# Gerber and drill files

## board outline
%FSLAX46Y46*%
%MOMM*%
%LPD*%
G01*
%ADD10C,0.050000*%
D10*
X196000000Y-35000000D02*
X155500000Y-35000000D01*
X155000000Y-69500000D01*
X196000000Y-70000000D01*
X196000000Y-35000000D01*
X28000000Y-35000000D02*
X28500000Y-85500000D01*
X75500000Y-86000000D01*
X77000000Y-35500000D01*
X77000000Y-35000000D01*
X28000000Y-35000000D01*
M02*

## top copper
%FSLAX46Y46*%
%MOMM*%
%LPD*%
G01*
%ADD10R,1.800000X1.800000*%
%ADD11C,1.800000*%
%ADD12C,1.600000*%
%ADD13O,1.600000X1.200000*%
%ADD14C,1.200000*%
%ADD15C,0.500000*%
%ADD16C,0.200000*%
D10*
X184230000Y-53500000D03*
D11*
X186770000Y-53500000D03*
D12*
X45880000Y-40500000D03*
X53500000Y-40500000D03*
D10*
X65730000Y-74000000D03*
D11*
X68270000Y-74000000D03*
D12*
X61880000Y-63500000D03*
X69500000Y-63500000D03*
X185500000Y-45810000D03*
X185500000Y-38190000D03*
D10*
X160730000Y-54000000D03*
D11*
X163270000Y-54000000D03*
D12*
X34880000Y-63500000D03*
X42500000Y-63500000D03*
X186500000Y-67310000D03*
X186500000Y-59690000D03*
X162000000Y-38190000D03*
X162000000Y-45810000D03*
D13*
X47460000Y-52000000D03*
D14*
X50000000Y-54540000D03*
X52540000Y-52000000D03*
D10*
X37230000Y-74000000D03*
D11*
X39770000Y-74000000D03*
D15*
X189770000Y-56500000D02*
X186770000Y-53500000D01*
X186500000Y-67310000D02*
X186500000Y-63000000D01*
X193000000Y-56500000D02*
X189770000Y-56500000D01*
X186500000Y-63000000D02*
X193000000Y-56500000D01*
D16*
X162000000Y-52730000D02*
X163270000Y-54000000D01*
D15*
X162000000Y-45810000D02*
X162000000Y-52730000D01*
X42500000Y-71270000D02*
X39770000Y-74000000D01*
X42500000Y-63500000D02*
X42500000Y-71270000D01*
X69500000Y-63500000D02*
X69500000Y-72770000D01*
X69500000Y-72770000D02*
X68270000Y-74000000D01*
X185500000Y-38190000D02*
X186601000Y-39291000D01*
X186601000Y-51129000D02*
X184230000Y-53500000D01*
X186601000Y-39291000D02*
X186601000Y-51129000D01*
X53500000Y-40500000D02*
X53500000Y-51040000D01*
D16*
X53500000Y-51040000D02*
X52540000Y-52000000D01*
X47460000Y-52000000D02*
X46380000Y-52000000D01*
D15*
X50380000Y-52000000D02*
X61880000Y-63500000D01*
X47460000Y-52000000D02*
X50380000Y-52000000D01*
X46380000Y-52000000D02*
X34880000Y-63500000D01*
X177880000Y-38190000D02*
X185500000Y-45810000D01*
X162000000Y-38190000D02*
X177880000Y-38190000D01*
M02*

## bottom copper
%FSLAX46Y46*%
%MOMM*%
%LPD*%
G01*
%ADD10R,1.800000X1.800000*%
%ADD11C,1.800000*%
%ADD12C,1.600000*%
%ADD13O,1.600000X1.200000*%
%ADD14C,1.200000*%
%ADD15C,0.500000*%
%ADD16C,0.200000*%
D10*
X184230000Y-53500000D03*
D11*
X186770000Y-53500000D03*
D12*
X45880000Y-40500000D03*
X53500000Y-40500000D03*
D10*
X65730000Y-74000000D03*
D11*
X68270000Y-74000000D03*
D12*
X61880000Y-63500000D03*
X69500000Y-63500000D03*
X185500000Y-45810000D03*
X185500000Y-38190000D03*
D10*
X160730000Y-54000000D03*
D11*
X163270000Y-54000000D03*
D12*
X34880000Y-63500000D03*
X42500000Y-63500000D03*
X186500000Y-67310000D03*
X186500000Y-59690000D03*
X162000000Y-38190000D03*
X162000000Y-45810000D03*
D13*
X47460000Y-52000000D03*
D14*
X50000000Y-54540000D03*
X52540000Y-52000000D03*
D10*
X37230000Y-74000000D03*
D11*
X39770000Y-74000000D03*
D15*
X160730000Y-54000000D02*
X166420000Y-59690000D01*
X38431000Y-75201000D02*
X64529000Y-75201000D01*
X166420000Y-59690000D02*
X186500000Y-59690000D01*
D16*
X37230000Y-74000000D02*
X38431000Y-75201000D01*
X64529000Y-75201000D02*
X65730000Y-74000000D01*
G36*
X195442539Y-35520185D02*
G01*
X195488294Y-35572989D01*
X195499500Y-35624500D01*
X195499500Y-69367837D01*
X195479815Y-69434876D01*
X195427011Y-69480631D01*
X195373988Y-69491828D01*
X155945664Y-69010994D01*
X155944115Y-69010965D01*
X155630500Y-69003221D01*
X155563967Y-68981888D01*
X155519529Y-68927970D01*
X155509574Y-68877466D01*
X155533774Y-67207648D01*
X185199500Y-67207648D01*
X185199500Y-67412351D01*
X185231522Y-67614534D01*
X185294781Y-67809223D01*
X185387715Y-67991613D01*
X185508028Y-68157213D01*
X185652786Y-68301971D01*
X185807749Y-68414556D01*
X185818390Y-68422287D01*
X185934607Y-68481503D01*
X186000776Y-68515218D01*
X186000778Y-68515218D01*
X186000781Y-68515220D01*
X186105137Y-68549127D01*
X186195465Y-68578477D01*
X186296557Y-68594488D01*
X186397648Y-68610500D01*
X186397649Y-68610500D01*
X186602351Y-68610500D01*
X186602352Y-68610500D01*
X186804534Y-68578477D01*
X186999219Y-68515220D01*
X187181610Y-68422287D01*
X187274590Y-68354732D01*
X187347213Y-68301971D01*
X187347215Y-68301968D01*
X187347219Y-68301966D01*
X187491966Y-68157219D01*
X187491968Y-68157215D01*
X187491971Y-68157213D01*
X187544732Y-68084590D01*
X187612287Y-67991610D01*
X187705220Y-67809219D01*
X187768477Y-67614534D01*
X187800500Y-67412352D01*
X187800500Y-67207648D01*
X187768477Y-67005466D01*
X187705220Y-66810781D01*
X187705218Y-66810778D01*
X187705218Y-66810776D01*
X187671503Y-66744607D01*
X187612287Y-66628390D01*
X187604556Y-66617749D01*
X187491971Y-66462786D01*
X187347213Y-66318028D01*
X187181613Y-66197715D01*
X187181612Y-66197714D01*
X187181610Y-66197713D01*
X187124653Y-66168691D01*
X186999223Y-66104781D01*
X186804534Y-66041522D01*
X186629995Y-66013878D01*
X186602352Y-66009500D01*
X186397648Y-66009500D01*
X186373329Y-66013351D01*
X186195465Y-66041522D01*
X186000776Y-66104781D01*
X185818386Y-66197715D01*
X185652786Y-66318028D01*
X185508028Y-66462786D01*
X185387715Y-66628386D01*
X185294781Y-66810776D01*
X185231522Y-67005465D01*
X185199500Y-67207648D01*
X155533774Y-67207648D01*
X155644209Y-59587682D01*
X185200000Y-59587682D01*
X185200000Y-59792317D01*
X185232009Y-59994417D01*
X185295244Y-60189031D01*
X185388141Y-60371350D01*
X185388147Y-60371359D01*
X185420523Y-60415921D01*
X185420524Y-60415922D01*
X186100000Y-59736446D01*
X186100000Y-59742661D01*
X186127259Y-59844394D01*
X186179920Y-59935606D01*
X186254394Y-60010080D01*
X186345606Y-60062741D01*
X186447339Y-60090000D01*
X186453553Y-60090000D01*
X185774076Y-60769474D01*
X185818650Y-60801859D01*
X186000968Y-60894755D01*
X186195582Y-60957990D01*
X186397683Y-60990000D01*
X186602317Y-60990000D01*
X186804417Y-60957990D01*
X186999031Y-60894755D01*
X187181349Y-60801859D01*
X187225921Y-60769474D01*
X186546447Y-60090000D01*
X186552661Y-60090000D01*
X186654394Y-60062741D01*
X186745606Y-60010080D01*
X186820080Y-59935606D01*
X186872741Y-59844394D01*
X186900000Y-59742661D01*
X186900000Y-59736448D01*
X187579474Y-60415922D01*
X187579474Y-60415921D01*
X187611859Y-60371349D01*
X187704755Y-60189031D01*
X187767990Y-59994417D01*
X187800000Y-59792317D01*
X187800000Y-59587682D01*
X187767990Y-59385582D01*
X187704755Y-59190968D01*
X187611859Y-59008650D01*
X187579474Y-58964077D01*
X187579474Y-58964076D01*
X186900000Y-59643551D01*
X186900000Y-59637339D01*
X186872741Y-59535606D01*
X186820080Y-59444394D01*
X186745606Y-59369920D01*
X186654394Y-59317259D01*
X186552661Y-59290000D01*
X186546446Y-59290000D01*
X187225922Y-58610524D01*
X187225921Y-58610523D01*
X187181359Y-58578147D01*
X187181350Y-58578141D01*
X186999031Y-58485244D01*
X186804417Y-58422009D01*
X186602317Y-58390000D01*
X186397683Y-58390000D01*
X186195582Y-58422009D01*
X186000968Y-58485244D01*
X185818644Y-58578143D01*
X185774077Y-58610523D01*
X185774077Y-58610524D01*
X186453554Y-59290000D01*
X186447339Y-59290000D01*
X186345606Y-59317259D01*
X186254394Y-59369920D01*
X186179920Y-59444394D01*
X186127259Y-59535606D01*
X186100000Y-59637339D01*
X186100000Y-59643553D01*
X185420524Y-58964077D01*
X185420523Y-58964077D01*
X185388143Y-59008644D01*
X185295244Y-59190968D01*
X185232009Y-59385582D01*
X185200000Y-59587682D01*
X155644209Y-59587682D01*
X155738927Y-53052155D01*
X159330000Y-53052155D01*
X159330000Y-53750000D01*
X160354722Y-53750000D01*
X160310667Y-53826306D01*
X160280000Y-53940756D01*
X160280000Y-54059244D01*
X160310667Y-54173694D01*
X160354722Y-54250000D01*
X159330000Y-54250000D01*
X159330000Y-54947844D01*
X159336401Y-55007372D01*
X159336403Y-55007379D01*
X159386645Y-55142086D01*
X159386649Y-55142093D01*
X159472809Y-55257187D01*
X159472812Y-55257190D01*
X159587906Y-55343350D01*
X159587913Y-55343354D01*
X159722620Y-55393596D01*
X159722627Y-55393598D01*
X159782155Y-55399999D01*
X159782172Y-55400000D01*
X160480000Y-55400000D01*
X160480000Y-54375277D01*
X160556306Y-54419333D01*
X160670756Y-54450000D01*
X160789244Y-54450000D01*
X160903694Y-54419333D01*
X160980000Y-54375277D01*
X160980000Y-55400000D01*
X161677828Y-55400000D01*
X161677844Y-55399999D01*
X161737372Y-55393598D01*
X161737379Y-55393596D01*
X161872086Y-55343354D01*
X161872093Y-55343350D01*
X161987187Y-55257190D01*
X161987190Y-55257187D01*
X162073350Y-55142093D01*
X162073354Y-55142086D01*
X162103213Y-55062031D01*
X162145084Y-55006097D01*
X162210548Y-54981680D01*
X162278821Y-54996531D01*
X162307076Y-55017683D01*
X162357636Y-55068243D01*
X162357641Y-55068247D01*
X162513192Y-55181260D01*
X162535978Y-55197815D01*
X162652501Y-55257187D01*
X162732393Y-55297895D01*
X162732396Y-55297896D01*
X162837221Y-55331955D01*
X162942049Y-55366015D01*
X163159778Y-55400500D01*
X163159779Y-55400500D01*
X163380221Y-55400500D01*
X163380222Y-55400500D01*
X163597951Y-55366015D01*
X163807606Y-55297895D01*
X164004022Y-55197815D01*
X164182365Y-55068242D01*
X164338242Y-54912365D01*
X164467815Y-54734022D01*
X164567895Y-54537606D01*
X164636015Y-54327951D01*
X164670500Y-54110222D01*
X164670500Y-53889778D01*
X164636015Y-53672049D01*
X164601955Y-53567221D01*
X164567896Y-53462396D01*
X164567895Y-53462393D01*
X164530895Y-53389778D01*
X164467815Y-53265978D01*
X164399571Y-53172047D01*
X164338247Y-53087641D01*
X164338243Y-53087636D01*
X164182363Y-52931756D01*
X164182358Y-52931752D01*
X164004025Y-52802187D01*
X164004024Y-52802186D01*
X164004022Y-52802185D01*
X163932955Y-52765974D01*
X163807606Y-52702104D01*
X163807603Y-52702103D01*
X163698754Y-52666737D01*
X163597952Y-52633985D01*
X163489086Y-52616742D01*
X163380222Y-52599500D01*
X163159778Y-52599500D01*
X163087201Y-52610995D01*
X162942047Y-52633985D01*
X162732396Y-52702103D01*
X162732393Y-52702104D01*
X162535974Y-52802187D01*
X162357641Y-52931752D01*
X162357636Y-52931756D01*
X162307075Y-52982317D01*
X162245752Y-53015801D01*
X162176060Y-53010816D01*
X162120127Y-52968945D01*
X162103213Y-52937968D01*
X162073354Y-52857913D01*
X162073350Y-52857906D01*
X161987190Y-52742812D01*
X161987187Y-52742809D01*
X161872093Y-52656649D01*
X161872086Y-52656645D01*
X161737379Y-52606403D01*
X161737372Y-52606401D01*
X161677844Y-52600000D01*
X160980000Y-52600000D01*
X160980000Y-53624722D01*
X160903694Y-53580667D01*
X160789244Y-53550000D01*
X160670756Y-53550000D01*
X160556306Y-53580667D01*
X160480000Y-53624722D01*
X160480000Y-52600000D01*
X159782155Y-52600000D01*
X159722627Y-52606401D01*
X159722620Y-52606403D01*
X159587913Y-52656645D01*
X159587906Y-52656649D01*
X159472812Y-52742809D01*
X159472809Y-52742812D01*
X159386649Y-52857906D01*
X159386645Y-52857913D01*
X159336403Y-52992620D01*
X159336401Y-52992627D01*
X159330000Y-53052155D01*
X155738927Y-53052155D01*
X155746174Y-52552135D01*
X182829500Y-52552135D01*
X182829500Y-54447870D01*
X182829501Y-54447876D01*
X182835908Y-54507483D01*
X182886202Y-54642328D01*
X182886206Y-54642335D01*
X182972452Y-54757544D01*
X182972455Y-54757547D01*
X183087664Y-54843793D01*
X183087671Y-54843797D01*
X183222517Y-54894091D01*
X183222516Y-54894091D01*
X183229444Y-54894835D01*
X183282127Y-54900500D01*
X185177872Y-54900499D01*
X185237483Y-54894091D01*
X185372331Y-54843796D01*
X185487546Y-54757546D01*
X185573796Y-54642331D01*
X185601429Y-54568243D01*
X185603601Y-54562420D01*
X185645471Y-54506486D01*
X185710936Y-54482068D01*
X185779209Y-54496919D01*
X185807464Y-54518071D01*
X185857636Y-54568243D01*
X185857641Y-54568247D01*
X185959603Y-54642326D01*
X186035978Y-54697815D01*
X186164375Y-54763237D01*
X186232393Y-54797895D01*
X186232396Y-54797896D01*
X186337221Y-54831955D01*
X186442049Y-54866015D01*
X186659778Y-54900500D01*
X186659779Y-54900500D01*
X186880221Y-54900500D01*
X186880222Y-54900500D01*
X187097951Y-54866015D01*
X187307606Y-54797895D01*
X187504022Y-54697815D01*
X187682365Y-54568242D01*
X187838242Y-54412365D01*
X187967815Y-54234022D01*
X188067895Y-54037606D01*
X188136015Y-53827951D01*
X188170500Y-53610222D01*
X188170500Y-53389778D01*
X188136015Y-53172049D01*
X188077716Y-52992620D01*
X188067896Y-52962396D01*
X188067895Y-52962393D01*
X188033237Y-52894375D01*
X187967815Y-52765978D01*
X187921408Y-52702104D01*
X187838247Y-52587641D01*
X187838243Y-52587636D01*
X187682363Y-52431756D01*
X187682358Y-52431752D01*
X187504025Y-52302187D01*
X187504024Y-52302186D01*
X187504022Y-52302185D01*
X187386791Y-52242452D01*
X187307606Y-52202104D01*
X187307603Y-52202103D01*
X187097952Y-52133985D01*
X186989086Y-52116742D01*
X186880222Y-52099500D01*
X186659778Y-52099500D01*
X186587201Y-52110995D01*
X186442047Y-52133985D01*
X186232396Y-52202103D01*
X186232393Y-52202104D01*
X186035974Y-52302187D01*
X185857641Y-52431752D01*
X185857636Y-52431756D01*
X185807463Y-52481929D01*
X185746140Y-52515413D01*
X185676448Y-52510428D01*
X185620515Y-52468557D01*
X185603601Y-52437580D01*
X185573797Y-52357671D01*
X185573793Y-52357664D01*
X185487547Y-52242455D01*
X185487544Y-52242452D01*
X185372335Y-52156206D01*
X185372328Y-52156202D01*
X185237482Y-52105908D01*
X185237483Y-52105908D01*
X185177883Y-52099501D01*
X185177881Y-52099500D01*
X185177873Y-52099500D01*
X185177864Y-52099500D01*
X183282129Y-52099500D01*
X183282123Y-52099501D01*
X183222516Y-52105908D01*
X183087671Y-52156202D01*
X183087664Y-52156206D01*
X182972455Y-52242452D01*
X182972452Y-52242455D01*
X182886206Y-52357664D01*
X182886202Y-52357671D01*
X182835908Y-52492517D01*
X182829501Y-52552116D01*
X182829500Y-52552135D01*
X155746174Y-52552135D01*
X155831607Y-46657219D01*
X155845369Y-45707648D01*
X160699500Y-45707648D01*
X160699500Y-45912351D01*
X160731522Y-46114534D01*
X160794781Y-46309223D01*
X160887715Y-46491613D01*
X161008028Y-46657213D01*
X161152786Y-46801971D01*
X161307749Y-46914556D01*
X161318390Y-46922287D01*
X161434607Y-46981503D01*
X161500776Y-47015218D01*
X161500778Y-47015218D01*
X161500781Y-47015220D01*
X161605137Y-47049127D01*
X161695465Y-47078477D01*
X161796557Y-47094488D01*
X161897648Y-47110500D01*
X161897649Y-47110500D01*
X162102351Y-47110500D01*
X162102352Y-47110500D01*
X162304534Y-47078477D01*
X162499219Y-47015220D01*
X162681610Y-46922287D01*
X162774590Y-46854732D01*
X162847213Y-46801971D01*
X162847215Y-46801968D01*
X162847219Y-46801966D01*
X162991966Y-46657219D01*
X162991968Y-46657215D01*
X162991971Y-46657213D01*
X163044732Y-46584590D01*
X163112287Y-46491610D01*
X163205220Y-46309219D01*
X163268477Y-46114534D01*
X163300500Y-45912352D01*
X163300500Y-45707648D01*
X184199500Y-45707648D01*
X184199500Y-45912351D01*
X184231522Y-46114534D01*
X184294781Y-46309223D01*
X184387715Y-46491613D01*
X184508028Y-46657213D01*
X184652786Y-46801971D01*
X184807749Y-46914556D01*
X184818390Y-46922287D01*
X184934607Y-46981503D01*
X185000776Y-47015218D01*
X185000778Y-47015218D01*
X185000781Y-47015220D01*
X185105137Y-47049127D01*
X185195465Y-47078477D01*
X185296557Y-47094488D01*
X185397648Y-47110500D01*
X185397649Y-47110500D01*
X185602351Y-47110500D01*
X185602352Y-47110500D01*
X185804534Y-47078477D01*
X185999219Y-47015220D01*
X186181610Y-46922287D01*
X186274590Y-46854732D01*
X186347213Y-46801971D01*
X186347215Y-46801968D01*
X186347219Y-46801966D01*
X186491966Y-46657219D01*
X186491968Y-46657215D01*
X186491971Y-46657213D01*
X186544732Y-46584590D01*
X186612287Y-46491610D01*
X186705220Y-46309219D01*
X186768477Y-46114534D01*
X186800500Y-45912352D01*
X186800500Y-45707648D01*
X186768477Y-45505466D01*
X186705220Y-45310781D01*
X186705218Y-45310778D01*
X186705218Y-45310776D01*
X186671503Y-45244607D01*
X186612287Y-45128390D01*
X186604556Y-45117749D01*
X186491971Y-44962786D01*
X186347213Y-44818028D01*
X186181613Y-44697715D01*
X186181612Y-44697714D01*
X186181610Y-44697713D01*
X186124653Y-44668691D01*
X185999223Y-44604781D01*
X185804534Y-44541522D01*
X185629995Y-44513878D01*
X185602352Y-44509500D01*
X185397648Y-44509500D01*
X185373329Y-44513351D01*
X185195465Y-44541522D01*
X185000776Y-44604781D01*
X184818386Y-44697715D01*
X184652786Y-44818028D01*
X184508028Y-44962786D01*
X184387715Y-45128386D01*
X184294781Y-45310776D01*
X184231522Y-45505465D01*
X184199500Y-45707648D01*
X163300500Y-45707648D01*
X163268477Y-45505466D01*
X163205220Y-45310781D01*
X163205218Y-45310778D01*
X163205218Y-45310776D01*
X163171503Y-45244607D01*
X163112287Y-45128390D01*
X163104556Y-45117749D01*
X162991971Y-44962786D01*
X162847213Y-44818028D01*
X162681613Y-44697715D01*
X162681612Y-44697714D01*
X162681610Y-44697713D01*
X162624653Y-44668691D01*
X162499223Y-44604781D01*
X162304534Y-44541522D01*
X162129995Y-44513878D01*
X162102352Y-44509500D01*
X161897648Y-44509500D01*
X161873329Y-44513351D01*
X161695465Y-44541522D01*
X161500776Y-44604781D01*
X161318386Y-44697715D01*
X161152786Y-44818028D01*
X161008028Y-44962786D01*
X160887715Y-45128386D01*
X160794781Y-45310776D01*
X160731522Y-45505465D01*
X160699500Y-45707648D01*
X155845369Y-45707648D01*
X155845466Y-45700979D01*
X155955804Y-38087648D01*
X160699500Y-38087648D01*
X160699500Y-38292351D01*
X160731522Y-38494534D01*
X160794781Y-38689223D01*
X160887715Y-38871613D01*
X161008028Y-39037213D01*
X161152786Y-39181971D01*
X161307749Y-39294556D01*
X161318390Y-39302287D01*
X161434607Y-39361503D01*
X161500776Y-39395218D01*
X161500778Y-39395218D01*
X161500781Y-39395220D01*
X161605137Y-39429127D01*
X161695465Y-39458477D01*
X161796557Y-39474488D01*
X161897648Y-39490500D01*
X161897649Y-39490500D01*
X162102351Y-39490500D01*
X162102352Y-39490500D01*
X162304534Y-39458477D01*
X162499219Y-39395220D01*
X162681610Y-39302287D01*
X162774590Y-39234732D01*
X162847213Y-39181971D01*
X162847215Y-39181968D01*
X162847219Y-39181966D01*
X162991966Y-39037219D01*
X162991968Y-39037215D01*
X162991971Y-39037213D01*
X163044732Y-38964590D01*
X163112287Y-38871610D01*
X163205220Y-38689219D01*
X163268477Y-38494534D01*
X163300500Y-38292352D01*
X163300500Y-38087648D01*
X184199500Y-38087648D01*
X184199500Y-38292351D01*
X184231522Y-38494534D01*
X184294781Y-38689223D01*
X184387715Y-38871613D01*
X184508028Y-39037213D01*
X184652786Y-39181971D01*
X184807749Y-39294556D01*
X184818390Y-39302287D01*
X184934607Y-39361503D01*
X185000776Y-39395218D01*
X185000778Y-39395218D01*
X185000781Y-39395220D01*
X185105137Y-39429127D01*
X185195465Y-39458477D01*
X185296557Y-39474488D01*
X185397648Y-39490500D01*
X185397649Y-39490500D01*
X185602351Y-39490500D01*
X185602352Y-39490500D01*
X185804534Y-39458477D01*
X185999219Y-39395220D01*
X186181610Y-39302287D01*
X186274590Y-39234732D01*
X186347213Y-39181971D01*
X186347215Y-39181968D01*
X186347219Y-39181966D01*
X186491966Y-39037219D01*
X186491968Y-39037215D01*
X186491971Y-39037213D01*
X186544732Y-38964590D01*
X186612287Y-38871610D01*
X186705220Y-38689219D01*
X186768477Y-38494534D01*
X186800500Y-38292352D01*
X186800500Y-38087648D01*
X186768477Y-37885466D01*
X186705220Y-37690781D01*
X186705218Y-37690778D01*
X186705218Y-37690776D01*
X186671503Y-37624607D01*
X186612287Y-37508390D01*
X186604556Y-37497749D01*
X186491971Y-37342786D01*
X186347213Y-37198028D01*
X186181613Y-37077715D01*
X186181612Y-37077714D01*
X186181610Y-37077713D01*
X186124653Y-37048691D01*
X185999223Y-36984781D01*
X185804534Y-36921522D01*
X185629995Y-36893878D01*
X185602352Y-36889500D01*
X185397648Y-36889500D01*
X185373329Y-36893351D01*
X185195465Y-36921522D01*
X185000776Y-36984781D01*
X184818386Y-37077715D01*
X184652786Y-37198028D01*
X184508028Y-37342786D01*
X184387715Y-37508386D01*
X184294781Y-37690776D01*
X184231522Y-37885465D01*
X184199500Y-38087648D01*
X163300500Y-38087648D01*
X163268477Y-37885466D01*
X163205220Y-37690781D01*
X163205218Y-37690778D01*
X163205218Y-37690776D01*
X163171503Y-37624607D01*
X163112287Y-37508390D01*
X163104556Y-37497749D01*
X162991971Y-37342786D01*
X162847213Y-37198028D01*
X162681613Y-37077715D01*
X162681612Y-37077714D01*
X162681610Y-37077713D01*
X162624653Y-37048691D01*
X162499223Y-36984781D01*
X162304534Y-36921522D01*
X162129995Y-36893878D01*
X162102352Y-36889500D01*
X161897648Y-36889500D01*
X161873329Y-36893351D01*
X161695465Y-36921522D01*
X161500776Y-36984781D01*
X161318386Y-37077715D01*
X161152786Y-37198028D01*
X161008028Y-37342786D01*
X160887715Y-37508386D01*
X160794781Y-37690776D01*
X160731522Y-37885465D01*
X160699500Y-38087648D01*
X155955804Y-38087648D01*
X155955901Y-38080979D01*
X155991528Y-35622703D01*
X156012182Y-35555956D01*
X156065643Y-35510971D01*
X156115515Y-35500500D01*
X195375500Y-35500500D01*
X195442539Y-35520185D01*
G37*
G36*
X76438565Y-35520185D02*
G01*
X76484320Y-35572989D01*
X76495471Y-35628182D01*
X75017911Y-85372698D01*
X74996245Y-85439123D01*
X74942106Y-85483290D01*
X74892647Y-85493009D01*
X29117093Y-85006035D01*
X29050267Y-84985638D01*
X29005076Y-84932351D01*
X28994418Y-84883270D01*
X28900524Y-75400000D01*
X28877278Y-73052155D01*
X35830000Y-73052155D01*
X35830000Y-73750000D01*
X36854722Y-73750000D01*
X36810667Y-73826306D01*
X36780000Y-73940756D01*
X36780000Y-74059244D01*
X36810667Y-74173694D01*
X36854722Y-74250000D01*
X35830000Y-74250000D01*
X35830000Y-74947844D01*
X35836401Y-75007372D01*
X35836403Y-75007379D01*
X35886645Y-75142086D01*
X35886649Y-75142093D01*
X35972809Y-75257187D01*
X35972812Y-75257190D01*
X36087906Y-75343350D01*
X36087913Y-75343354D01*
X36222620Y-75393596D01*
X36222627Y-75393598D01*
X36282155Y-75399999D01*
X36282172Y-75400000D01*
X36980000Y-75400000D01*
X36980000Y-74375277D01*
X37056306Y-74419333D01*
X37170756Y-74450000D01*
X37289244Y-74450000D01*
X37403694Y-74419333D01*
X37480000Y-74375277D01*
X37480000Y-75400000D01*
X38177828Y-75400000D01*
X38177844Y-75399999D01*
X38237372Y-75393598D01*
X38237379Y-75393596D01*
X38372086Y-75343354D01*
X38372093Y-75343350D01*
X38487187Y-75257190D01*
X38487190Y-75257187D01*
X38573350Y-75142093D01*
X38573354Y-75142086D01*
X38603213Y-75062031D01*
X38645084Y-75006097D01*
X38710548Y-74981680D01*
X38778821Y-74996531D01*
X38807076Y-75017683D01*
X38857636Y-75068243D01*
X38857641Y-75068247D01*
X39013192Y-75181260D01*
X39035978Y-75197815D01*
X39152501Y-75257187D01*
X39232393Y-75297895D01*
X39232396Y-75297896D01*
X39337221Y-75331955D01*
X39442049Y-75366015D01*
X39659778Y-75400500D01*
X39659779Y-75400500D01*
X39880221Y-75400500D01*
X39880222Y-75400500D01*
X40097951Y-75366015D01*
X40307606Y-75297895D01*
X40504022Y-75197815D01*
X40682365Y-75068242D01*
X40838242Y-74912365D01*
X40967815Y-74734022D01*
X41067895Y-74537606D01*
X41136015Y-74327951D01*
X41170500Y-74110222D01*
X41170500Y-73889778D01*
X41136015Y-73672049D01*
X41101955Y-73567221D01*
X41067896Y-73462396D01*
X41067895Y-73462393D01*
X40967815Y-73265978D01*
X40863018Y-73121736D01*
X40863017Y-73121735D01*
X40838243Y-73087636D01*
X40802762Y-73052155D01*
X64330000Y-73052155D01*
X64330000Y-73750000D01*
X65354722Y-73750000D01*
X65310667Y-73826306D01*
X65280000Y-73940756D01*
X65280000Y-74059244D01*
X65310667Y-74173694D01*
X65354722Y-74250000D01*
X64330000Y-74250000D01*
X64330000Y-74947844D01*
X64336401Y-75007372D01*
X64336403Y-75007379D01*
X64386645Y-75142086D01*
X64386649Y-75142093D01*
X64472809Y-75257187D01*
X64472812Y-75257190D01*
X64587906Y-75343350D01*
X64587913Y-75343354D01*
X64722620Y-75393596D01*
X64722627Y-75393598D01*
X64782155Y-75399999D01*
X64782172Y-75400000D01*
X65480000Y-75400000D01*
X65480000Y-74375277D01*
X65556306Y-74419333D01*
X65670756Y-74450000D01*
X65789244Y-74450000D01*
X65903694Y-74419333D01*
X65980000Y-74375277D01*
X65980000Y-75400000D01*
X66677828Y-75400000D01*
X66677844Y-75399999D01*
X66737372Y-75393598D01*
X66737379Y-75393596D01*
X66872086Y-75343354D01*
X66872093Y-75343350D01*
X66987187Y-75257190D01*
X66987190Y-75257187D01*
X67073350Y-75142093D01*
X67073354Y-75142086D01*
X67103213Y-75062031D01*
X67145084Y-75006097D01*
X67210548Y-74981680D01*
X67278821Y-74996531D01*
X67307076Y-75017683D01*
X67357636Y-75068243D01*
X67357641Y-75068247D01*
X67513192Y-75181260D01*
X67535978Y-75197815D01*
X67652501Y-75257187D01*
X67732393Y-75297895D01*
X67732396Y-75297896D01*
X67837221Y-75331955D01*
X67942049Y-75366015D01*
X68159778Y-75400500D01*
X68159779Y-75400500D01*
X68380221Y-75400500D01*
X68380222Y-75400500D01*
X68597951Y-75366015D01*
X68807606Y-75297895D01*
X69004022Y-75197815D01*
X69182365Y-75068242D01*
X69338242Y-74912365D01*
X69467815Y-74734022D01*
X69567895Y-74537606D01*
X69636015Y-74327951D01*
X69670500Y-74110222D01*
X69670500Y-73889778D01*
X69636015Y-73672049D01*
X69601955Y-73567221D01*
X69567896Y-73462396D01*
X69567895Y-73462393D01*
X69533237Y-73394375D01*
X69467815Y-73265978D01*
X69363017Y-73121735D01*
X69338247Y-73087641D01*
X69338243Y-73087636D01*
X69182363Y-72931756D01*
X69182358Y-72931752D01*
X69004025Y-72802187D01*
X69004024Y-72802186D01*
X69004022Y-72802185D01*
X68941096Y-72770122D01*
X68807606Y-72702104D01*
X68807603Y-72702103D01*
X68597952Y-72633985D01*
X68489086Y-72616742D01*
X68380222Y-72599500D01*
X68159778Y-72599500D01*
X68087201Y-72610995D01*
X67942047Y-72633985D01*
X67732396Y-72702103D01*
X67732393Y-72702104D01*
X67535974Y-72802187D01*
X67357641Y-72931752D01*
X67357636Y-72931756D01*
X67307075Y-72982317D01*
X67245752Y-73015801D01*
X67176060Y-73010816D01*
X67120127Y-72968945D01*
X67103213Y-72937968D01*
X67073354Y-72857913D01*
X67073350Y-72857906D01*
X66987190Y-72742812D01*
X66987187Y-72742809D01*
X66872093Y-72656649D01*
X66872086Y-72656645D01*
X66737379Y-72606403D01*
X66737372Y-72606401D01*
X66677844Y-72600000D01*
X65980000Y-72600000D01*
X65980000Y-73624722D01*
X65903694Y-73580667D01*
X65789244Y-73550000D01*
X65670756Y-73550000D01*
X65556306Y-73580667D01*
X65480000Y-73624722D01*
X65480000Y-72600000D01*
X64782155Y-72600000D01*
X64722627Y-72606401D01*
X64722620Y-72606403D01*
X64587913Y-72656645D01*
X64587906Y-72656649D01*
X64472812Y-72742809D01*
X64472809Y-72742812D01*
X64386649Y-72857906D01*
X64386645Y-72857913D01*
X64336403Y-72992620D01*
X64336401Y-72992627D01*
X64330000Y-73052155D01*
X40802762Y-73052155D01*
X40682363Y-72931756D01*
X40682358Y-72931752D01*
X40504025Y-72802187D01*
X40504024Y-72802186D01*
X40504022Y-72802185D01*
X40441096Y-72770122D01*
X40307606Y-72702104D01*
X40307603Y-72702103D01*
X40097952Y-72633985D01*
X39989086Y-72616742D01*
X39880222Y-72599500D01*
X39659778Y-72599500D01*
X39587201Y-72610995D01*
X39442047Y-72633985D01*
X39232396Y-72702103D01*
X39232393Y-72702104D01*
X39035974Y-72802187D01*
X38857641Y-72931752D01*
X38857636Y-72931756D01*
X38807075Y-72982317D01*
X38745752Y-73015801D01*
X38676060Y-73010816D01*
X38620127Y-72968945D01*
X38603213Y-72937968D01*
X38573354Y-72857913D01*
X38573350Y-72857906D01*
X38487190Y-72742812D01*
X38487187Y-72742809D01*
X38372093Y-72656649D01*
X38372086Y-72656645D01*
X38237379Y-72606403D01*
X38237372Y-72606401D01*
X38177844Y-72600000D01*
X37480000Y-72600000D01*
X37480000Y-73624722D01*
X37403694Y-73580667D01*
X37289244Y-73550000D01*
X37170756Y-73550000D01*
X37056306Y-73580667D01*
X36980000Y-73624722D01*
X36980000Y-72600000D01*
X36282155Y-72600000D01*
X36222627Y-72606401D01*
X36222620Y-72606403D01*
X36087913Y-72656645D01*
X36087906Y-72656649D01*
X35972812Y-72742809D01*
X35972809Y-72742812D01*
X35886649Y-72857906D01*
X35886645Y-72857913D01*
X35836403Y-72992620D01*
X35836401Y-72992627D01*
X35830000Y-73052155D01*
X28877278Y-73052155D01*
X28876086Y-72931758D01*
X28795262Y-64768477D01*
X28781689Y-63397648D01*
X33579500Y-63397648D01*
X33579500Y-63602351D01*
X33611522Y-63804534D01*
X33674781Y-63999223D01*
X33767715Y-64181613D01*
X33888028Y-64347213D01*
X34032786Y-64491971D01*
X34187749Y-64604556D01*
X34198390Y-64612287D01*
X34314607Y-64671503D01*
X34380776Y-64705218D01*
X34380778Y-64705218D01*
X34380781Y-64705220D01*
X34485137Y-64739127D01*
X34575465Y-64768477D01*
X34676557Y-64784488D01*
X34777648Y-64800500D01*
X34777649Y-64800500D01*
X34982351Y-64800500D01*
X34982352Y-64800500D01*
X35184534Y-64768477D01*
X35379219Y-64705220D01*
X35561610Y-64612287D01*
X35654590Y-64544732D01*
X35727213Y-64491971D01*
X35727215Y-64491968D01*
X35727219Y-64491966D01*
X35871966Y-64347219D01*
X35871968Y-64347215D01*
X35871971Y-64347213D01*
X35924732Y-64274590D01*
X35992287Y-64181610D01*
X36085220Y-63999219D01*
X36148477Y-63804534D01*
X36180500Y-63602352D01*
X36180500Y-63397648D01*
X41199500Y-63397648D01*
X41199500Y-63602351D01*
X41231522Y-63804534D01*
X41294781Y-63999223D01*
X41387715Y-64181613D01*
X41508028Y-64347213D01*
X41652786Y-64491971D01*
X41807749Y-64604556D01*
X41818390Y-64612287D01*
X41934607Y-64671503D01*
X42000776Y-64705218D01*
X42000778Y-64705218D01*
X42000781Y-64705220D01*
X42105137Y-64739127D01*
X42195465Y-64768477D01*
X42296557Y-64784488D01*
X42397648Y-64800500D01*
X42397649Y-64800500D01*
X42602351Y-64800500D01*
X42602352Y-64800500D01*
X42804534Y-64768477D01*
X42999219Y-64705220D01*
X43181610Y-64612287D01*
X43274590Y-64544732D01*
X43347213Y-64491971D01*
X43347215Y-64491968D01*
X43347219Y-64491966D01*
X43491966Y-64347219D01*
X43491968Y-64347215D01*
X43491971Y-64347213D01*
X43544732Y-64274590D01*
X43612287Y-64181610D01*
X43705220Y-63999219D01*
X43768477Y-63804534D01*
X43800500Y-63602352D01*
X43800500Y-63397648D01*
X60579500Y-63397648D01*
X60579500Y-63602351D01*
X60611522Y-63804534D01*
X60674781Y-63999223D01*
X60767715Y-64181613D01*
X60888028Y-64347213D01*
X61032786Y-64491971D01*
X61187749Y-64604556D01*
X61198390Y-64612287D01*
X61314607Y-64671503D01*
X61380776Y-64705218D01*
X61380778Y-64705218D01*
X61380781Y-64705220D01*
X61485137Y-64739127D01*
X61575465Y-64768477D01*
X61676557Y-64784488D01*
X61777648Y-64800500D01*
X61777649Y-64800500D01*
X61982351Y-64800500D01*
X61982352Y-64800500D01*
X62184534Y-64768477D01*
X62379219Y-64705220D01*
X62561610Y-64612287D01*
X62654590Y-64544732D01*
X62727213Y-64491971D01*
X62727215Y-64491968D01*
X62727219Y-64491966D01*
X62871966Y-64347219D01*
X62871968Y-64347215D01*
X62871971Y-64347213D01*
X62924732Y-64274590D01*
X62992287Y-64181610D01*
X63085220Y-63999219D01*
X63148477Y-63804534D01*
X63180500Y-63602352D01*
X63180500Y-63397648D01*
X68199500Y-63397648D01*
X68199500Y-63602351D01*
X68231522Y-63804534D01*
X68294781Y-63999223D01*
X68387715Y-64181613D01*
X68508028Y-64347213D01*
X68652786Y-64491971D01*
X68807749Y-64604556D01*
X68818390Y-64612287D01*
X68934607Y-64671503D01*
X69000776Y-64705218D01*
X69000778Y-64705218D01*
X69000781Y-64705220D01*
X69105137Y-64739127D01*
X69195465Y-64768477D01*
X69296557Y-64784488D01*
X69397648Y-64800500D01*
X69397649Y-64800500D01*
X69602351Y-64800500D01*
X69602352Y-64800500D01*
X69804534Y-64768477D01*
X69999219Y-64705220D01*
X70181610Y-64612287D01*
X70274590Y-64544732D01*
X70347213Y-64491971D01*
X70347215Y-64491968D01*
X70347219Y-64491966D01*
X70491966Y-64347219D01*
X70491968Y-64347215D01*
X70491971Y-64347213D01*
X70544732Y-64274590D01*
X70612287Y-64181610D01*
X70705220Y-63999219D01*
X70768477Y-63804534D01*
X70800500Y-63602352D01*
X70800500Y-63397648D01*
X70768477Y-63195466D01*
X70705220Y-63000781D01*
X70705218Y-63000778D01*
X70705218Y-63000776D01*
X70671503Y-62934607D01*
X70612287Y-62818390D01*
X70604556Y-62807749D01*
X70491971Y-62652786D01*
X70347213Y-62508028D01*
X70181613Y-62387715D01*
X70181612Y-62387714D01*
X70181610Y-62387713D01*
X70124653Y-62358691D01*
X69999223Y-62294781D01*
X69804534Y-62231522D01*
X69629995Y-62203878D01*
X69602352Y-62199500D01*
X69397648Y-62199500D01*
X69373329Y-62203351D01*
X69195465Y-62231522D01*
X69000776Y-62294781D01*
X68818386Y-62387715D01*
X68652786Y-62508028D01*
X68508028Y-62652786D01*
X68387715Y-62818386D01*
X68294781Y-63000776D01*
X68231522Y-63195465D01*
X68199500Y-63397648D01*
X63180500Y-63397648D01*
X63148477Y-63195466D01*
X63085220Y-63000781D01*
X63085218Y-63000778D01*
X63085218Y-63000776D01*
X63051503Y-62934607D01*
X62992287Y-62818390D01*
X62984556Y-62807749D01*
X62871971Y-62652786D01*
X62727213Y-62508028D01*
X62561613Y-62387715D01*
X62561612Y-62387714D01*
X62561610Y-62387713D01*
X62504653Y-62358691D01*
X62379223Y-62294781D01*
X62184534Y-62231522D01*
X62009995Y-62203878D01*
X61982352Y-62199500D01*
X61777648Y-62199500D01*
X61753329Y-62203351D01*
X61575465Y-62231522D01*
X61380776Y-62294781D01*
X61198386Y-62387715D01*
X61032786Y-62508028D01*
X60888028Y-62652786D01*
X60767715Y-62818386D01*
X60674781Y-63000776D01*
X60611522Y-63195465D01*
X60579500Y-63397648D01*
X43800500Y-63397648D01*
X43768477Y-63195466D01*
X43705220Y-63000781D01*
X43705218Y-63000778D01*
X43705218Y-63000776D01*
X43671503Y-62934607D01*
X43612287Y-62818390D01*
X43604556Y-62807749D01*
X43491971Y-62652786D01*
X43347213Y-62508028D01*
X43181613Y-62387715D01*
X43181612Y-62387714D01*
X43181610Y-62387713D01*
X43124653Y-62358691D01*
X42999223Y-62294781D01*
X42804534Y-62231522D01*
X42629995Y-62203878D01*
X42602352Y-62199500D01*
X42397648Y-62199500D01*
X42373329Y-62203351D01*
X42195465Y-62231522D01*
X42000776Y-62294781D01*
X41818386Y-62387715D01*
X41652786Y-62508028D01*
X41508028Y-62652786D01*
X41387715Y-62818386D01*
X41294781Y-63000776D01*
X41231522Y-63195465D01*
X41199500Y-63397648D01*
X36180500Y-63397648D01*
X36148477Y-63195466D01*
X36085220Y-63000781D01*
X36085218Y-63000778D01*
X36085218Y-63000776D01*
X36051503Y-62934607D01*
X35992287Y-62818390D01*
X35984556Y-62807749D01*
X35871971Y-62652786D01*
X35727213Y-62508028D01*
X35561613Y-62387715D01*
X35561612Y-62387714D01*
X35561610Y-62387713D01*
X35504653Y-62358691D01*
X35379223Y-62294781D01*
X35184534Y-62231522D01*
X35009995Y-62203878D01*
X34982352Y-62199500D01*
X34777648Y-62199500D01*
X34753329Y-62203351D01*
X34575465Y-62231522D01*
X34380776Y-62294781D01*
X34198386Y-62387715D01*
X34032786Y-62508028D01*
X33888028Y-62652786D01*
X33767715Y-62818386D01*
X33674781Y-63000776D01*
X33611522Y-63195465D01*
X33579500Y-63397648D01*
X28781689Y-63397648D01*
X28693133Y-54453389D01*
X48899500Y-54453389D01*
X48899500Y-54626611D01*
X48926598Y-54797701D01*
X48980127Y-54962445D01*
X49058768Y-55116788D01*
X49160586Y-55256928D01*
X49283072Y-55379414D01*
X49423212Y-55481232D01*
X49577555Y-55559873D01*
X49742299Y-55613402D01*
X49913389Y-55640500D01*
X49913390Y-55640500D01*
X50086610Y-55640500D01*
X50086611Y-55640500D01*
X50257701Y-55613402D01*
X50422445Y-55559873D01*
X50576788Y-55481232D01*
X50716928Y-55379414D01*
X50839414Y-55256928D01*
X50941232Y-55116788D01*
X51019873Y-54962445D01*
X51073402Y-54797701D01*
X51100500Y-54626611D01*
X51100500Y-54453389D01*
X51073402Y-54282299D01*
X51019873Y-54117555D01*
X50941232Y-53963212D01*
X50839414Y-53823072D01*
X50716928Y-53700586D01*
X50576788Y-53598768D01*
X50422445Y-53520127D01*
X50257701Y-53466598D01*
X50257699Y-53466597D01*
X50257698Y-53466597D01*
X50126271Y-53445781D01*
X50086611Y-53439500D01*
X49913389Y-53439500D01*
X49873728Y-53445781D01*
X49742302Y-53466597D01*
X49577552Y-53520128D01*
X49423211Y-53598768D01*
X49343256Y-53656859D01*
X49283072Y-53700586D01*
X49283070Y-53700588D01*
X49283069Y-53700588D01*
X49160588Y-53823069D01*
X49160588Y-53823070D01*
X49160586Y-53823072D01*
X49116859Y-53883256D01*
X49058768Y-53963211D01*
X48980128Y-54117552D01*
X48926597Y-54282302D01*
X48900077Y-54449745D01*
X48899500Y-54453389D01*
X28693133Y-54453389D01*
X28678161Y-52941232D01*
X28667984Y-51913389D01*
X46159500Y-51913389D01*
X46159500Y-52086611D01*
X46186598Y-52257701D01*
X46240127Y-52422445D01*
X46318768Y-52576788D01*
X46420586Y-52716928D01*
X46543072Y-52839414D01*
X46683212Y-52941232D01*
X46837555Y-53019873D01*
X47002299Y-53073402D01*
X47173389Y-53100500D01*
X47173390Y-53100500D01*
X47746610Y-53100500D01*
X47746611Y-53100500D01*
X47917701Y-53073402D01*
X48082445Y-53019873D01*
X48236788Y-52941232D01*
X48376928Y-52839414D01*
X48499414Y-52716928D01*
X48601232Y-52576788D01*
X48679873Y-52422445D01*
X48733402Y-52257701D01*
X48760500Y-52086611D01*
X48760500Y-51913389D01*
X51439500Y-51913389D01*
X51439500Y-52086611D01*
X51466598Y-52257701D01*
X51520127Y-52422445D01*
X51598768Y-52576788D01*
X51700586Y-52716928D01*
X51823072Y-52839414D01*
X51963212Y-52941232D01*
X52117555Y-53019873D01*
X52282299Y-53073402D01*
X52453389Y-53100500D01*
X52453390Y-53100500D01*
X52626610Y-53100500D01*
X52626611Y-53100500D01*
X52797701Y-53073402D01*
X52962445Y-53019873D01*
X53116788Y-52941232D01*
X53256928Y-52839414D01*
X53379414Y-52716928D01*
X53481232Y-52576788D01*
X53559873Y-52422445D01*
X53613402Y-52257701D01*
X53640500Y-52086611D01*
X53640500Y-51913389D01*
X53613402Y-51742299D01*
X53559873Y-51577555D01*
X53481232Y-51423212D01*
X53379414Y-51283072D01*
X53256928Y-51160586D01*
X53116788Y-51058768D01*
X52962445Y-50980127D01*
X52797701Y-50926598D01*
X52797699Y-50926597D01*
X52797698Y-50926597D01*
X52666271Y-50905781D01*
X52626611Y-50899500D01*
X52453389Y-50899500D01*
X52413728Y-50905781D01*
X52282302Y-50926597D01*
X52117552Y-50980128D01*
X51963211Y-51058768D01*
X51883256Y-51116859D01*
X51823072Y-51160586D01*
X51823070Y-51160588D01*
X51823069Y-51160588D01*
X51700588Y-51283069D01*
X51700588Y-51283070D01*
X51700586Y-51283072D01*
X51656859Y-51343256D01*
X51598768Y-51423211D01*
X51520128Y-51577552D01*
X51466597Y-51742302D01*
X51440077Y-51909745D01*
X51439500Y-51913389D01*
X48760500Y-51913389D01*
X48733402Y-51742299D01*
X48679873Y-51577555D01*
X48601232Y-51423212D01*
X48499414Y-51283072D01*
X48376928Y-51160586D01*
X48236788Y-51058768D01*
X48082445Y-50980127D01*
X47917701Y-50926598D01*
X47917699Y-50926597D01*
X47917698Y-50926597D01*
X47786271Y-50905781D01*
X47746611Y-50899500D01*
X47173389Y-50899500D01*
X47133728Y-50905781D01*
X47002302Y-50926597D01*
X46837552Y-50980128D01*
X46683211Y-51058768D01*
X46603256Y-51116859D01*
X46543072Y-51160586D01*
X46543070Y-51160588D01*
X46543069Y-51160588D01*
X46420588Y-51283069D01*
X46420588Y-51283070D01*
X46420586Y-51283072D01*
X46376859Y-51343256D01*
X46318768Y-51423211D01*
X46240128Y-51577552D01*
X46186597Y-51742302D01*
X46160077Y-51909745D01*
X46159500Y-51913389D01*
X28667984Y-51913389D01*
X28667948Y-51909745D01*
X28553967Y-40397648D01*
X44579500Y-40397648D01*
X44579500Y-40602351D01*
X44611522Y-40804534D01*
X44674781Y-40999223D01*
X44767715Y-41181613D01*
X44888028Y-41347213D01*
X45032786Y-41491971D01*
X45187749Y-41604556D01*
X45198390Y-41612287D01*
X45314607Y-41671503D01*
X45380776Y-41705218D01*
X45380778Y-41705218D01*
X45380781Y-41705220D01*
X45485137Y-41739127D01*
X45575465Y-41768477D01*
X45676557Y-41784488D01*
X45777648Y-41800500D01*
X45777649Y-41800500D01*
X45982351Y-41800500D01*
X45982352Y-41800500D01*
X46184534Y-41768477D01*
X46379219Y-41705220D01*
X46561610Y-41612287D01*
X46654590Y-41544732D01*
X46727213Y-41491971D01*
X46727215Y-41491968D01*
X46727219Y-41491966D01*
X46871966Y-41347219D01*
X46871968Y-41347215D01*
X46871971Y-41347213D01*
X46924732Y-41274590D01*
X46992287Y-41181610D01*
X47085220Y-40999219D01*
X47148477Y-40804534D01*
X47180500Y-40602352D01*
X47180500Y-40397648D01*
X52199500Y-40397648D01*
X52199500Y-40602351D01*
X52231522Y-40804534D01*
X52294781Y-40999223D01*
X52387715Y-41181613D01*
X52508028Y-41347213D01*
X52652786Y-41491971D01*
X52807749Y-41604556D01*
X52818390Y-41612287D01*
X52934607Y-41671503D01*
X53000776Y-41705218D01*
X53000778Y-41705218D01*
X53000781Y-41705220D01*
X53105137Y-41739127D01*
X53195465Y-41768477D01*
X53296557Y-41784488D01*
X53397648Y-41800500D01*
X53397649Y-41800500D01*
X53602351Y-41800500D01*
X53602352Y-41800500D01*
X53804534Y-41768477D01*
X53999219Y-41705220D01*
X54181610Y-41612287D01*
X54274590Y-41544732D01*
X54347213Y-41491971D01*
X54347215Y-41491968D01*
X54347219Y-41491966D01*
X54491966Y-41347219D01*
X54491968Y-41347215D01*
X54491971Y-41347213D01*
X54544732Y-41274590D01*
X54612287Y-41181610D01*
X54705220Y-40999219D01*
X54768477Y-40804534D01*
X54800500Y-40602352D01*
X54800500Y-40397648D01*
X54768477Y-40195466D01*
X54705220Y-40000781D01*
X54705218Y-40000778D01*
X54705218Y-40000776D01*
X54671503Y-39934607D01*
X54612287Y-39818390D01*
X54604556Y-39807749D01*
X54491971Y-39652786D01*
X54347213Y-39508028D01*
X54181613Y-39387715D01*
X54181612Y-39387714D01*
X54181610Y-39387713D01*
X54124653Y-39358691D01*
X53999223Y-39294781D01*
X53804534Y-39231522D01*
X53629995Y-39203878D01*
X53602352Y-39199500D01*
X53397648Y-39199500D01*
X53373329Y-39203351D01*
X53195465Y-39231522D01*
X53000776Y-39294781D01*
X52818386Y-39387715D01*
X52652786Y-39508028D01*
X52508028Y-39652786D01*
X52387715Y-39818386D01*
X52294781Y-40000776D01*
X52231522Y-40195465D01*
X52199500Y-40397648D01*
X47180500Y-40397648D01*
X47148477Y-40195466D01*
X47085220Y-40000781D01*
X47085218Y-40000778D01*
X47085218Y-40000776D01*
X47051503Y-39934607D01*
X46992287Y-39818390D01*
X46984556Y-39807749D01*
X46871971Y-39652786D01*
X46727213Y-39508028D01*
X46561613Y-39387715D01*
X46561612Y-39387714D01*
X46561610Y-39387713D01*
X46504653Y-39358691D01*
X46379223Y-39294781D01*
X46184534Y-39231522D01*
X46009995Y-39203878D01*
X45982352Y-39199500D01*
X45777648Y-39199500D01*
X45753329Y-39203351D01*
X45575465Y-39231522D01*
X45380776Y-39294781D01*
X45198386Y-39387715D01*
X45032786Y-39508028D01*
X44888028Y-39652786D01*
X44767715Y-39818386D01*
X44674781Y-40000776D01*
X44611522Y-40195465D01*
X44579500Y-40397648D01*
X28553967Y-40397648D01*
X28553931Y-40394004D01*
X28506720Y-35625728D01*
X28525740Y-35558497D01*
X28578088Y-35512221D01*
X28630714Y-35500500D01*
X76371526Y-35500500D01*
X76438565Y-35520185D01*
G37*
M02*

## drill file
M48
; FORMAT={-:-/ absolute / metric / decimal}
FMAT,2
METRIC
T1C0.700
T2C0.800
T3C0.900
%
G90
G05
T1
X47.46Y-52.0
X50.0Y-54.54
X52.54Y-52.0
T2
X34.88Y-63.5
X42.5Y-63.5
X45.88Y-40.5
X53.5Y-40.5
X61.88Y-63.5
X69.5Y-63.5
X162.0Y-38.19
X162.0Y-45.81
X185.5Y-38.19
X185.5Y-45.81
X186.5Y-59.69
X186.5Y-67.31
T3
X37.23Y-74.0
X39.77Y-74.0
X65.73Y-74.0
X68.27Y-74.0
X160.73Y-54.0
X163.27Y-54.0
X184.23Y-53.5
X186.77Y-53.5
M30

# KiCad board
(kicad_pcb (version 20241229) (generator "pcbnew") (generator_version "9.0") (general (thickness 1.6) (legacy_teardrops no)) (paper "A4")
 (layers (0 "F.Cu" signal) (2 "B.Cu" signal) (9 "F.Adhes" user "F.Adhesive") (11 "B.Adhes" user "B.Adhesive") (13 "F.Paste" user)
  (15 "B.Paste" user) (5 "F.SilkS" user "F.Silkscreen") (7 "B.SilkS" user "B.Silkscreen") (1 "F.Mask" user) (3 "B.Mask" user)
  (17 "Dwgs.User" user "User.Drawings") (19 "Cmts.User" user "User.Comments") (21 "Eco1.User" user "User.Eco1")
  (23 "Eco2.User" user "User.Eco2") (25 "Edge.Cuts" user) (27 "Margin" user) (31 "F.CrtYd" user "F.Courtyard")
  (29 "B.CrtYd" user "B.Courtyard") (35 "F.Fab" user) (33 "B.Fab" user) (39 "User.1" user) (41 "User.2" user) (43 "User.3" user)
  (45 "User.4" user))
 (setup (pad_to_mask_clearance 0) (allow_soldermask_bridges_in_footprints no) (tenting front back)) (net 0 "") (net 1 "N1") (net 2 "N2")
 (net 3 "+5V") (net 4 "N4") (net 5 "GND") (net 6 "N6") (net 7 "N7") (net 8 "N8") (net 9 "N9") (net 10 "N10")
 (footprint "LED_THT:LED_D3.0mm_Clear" (layer "F.Cu") (at 184.23 53.5)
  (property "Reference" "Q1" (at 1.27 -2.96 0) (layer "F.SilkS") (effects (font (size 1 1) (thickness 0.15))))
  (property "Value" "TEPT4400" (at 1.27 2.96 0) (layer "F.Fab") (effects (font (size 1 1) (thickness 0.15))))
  (pad "1" thru_hole rect (at 0 0) (size 1.8 1.8) (drill 0.9) (layers "*.Cu" "*.Mask") (remove_unused_layers no) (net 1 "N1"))
  (pad "2" thru_hole circle (at 2.54 0) (size 1.8 1.8) (drill 0.9) (layers "*.Cu" "*.Mask") (remove_unused_layers no) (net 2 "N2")))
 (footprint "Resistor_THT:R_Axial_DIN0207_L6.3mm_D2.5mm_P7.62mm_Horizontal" (layer "F.Cu") (at 45.88 40.5)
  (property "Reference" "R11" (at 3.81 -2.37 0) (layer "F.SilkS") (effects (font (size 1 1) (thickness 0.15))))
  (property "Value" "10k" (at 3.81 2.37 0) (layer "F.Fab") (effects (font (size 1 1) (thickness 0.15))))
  (pad "1" thru_hole circle (at 0 0) (size 1.6 1.6) (drill 0.8) (layers "*.Cu" "*.Mask") (remove_unused_layers no) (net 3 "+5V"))
  (pad "2" thru_hole circle (at 7.62 0) (size 1.6 1.6) (drill 0.8) (layers "*.Cu" "*.Mask") (remove_unused_layers no) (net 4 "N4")))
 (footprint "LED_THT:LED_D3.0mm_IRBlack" (layer "F.Cu") (at 65.73 74)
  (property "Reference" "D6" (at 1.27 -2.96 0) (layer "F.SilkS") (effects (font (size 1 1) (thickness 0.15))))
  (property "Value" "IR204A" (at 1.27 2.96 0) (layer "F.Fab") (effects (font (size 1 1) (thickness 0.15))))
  (pad "1" thru_hole rect (at 0 0) (size 1.8 1.8) (drill 0.9) (layers "*.Cu" "*.Mask") (remove_unused_layers no) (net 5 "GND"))
  (pad "2" thru_hole circle (at 2.54 0) (size 1.8 1.8) (drill 0.9) (layers "*.Cu" "*.Mask") (remove_unused_layers no) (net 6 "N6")))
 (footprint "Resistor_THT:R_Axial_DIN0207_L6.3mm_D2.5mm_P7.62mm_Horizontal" (layer "F.Cu") (at 61.88 63.5)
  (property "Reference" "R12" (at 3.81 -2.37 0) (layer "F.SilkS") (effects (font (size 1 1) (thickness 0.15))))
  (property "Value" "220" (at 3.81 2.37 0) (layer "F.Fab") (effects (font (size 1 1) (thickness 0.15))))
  (pad "1" thru_hole circle (at 0 0) (size 1.6 1.6) (drill 0.8) (layers "*.Cu" "*.Mask") (remove_unused_layers no) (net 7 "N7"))
  (pad "2" thru_hole circle (at 7.62 0) (size 1.6 1.6) (drill 0.8) (layers "*.Cu" "*.Mask") (remove_unused_layers no) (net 6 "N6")))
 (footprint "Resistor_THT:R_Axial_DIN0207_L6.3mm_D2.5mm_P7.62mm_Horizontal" (layer "F.Cu") (at 185.5 45.81 90)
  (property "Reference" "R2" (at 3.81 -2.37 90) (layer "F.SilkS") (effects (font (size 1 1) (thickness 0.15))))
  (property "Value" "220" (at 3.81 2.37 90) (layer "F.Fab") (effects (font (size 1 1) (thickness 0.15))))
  (pad "1" thru_hole circle (at 0 0 90) (size 1.6 1.6) (drill 0.8) (layers "*.Cu" "*.Mask") (remove_unused_layers no) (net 3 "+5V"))
  (pad "2" thru_hole circle (at 7.62 0 90) (size 1.6 1.6) (drill 0.8) (layers "*.Cu" "*.Mask") (remove_unused_layers no) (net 1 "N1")))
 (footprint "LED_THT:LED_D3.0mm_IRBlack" (layer "F.Cu") (at 160.73 54)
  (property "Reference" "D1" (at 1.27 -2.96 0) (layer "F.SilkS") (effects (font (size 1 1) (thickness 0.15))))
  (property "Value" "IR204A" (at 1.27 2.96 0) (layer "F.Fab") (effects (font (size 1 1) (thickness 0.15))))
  (pad "1" thru_hole rect (at 0 0) (size 1.8 1.8) (drill 0.9) (layers "*.Cu" "*.Mask") (remove_unused_layers no) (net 5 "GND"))
  (pad "2" thru_hole circle (at 2.54 0) (size 1.8 1.8) (drill 0.9) (layers "*.Cu" "*.Mask") (remove_unused_layers no) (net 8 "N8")))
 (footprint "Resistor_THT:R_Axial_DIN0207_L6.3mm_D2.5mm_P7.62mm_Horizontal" (layer "F.Cu") (at 34.88 63.5)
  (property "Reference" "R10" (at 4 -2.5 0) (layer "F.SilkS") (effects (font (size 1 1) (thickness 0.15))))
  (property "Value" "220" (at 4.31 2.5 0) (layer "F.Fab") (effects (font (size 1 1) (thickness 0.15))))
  (pad "1" thru_hole circle (at 0 0) (size 1.6 1.6) (drill 0.8) (layers "*.Cu" "*.Mask") (remove_unused_layers no) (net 7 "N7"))
  (pad "2" thru_hole circle (at 7.62 0) (size 1.6 1.6) (drill 0.8) (layers "*.Cu" "*.Mask") (remove_unused_layers no) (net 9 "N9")))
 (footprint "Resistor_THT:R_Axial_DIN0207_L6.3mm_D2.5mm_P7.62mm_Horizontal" (layer "F.Cu") (at 186.5 67.31 90)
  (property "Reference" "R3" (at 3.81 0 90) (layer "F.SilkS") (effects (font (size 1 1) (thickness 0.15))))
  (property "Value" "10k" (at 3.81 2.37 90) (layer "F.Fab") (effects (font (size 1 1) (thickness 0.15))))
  (pad "1" thru_hole circle (at 0 0 90) (size 1.6 1.6) (drill 0.8) (layers "*.Cu" "*.Mask") (remove_unused_layers no) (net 2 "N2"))
  (pad "2" thru_hole circle (at 7.62 0 90) (size 1.6 1.6) (drill 0.8) (layers "*.Cu" "*.Mask") (remove_unused_layers no) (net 5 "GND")))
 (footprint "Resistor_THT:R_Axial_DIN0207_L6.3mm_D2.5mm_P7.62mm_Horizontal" (layer "F.Cu") (at 162 38.19 -90)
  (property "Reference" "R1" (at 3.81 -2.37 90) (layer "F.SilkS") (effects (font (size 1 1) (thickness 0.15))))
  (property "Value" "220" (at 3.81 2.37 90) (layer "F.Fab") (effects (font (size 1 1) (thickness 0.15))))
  (pad "1" thru_hole circle (at 0 0 270) (size 1.6 1.6) (drill 0.8) (layers "*.Cu" "*.Mask") (remove_unused_layers no) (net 3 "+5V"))
  (pad "2" thru_hole circle (at 7.62 0 270) (size 1.6 1.6) (drill 0.8) (layers "*.Cu" "*.Mask") (remove_unused_layers no) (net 8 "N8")))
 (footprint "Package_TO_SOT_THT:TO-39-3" (layer "F.Cu") (at 47.46 52)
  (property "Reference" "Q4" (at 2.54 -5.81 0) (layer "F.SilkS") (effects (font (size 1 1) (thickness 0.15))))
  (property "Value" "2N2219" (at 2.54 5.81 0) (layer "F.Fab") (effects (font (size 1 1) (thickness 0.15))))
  (pad "1" thru_hole oval (at 0 0) (size 1.6 1.2) (drill 0.7) (layers "*.Cu" "*.Mask") (remove_unused_layers no) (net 7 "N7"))
  (pad "2" thru_hole circle (at 2.54 2.54) (size 1.2 1.2) (drill 0.7) (layers "*.Cu" "*.Mask") (remove_unused_layers no) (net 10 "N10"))
  (pad "3" thru_hole circle (at 5.08 0) (size 1.2 1.2) (drill 0.7) (layers "*.Cu" "*.Mask") (remove_unused_layers no) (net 4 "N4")))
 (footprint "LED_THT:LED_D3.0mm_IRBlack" (layer "F.Cu") (at 37.23 74)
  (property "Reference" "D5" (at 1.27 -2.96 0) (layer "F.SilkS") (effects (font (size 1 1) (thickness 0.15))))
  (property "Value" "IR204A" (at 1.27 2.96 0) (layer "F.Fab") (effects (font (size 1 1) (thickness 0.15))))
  (pad "1" thru_hole rect (at 0 0) (size 1.8 1.8) (drill 0.9) (layers "*.Cu" "*.Mask") (remove_unused_layers no) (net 5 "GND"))
  (pad "2" thru_hole circle (at 2.54 0) (size 1.8 1.8) (drill 0.9) (layers "*.Cu" "*.Mask") (remove_unused_layers no) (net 9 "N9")))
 (gr_poly (pts (xy 196 35) (xy 155.5 35) (xy 155 69.5) (xy 196 70)) (stroke (width 0.05) (type solid)) (fill no) (layer "Edge.Cuts"))
 (gr_poly
  (pts (xy 28 35) (xy 28.5 85.5) (xy 75.5 86) (xy 77 35.5) (xy 77 35)) (stroke (width 0.05) (type solid)) (fill no) (layer "Edge.Cuts"))
 (segment (start 189.77 56.5) (end 186.77 53.5) (width 0.5) (layer "F.Cu") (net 2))
 (segment (start 186.5 67.31) (end 186.5 63) (width 0.5) (layer "F.Cu") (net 2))
 (segment (start 193 56.5) (end 189.77 56.5) (width 0.5) (layer "F.Cu") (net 2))
 (segment (start 186.5 63) (end 193 56.5) (width 0.5) (layer "F.Cu") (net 2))
 (segment (start 162 52.73) (end 163.27 54) (width 0.2) (layer "F.Cu") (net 8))
 (segment (start 162 45.81) (end 162 52.73) (width 0.5) (layer "F.Cu") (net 8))
 (segment (start 160.73 54) (end 166.42 59.69) (width 0.5) (layer "B.Cu") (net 5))
 (segment (start 38.431 75.201) (end 64.529 75.201) (width 0.5) (layer "B.Cu") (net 5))
 (segment (start 166.42 59.69) (end 186.5 59.69) (width 0.5) (layer "B.Cu") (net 5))
 (segment (start 37.23 74) (end 38.431 75.201) (width 0.2) (layer "B.Cu") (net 5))
 (segment (start 64.529 75.201) (end 65.73 74) (width 0.2) (layer "B.Cu") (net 5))
 (segment (start 42.5 71.27) (end 39.77 74) (width 0.5) (layer "F.Cu") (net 9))
 (segment (start 42.5 63.5) (end 42.5 71.27) (width 0.5) (layer "F.Cu") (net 9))
 (segment (start 69.5 63.5) (end 69.5 72.77) (width 0.5) (layer "F.Cu") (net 6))
 (segment (start 69.5 72.77) (end 68.27 74) (width 0.5) (layer "F.Cu") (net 6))
 (segment (start 185.5 38.19) (end 186.601 39.291) (width 0.5) (layer "F.Cu") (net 1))
 (segment (start 186.601 51.129) (end 184.23 53.5) (width 0.5) (layer "F.Cu") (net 1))
 (segment (start 186.601 39.291) (end 186.601 51.129) (width 0.5) (layer "F.Cu") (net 1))
 (segment (start 53.5 40.5) (end 53.5 51.04) (width 0.5) (layer "F.Cu") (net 4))
 (segment (start 53.5 51.04) (end 52.54 52) (width 0.2) (layer "F.Cu") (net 4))
 (segment (start 47.46 52) (end 46.38 52) (width 0.2) (layer "F.Cu") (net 7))
 (segment (start 50.38 52) (end 61.88 63.5) (width 0.5) (layer "F.Cu") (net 7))
 (segment (start 47.46 52) (end 50.38 52) (width 0.5) (layer "F.Cu") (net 7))
 (segment (start 46.38 52) (end 34.88 63.5) (width 0.5) (layer "F.Cu") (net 7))
 (segment (start 177.88 38.19) (end 185.5 45.81) (width 0.5) (layer "F.Cu") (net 3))
 (segment (start 162 38.19) (end 177.88 38.19) (width 0.5) (layer "F.Cu") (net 3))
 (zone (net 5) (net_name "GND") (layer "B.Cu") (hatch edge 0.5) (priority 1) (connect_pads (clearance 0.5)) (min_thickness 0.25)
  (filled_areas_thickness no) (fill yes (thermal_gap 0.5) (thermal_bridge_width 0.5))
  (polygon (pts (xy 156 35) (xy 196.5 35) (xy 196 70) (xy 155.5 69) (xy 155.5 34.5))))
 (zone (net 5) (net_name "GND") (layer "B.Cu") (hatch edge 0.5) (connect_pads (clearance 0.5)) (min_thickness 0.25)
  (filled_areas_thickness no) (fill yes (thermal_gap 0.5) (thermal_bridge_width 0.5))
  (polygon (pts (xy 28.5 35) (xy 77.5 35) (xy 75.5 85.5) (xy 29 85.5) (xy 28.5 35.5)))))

